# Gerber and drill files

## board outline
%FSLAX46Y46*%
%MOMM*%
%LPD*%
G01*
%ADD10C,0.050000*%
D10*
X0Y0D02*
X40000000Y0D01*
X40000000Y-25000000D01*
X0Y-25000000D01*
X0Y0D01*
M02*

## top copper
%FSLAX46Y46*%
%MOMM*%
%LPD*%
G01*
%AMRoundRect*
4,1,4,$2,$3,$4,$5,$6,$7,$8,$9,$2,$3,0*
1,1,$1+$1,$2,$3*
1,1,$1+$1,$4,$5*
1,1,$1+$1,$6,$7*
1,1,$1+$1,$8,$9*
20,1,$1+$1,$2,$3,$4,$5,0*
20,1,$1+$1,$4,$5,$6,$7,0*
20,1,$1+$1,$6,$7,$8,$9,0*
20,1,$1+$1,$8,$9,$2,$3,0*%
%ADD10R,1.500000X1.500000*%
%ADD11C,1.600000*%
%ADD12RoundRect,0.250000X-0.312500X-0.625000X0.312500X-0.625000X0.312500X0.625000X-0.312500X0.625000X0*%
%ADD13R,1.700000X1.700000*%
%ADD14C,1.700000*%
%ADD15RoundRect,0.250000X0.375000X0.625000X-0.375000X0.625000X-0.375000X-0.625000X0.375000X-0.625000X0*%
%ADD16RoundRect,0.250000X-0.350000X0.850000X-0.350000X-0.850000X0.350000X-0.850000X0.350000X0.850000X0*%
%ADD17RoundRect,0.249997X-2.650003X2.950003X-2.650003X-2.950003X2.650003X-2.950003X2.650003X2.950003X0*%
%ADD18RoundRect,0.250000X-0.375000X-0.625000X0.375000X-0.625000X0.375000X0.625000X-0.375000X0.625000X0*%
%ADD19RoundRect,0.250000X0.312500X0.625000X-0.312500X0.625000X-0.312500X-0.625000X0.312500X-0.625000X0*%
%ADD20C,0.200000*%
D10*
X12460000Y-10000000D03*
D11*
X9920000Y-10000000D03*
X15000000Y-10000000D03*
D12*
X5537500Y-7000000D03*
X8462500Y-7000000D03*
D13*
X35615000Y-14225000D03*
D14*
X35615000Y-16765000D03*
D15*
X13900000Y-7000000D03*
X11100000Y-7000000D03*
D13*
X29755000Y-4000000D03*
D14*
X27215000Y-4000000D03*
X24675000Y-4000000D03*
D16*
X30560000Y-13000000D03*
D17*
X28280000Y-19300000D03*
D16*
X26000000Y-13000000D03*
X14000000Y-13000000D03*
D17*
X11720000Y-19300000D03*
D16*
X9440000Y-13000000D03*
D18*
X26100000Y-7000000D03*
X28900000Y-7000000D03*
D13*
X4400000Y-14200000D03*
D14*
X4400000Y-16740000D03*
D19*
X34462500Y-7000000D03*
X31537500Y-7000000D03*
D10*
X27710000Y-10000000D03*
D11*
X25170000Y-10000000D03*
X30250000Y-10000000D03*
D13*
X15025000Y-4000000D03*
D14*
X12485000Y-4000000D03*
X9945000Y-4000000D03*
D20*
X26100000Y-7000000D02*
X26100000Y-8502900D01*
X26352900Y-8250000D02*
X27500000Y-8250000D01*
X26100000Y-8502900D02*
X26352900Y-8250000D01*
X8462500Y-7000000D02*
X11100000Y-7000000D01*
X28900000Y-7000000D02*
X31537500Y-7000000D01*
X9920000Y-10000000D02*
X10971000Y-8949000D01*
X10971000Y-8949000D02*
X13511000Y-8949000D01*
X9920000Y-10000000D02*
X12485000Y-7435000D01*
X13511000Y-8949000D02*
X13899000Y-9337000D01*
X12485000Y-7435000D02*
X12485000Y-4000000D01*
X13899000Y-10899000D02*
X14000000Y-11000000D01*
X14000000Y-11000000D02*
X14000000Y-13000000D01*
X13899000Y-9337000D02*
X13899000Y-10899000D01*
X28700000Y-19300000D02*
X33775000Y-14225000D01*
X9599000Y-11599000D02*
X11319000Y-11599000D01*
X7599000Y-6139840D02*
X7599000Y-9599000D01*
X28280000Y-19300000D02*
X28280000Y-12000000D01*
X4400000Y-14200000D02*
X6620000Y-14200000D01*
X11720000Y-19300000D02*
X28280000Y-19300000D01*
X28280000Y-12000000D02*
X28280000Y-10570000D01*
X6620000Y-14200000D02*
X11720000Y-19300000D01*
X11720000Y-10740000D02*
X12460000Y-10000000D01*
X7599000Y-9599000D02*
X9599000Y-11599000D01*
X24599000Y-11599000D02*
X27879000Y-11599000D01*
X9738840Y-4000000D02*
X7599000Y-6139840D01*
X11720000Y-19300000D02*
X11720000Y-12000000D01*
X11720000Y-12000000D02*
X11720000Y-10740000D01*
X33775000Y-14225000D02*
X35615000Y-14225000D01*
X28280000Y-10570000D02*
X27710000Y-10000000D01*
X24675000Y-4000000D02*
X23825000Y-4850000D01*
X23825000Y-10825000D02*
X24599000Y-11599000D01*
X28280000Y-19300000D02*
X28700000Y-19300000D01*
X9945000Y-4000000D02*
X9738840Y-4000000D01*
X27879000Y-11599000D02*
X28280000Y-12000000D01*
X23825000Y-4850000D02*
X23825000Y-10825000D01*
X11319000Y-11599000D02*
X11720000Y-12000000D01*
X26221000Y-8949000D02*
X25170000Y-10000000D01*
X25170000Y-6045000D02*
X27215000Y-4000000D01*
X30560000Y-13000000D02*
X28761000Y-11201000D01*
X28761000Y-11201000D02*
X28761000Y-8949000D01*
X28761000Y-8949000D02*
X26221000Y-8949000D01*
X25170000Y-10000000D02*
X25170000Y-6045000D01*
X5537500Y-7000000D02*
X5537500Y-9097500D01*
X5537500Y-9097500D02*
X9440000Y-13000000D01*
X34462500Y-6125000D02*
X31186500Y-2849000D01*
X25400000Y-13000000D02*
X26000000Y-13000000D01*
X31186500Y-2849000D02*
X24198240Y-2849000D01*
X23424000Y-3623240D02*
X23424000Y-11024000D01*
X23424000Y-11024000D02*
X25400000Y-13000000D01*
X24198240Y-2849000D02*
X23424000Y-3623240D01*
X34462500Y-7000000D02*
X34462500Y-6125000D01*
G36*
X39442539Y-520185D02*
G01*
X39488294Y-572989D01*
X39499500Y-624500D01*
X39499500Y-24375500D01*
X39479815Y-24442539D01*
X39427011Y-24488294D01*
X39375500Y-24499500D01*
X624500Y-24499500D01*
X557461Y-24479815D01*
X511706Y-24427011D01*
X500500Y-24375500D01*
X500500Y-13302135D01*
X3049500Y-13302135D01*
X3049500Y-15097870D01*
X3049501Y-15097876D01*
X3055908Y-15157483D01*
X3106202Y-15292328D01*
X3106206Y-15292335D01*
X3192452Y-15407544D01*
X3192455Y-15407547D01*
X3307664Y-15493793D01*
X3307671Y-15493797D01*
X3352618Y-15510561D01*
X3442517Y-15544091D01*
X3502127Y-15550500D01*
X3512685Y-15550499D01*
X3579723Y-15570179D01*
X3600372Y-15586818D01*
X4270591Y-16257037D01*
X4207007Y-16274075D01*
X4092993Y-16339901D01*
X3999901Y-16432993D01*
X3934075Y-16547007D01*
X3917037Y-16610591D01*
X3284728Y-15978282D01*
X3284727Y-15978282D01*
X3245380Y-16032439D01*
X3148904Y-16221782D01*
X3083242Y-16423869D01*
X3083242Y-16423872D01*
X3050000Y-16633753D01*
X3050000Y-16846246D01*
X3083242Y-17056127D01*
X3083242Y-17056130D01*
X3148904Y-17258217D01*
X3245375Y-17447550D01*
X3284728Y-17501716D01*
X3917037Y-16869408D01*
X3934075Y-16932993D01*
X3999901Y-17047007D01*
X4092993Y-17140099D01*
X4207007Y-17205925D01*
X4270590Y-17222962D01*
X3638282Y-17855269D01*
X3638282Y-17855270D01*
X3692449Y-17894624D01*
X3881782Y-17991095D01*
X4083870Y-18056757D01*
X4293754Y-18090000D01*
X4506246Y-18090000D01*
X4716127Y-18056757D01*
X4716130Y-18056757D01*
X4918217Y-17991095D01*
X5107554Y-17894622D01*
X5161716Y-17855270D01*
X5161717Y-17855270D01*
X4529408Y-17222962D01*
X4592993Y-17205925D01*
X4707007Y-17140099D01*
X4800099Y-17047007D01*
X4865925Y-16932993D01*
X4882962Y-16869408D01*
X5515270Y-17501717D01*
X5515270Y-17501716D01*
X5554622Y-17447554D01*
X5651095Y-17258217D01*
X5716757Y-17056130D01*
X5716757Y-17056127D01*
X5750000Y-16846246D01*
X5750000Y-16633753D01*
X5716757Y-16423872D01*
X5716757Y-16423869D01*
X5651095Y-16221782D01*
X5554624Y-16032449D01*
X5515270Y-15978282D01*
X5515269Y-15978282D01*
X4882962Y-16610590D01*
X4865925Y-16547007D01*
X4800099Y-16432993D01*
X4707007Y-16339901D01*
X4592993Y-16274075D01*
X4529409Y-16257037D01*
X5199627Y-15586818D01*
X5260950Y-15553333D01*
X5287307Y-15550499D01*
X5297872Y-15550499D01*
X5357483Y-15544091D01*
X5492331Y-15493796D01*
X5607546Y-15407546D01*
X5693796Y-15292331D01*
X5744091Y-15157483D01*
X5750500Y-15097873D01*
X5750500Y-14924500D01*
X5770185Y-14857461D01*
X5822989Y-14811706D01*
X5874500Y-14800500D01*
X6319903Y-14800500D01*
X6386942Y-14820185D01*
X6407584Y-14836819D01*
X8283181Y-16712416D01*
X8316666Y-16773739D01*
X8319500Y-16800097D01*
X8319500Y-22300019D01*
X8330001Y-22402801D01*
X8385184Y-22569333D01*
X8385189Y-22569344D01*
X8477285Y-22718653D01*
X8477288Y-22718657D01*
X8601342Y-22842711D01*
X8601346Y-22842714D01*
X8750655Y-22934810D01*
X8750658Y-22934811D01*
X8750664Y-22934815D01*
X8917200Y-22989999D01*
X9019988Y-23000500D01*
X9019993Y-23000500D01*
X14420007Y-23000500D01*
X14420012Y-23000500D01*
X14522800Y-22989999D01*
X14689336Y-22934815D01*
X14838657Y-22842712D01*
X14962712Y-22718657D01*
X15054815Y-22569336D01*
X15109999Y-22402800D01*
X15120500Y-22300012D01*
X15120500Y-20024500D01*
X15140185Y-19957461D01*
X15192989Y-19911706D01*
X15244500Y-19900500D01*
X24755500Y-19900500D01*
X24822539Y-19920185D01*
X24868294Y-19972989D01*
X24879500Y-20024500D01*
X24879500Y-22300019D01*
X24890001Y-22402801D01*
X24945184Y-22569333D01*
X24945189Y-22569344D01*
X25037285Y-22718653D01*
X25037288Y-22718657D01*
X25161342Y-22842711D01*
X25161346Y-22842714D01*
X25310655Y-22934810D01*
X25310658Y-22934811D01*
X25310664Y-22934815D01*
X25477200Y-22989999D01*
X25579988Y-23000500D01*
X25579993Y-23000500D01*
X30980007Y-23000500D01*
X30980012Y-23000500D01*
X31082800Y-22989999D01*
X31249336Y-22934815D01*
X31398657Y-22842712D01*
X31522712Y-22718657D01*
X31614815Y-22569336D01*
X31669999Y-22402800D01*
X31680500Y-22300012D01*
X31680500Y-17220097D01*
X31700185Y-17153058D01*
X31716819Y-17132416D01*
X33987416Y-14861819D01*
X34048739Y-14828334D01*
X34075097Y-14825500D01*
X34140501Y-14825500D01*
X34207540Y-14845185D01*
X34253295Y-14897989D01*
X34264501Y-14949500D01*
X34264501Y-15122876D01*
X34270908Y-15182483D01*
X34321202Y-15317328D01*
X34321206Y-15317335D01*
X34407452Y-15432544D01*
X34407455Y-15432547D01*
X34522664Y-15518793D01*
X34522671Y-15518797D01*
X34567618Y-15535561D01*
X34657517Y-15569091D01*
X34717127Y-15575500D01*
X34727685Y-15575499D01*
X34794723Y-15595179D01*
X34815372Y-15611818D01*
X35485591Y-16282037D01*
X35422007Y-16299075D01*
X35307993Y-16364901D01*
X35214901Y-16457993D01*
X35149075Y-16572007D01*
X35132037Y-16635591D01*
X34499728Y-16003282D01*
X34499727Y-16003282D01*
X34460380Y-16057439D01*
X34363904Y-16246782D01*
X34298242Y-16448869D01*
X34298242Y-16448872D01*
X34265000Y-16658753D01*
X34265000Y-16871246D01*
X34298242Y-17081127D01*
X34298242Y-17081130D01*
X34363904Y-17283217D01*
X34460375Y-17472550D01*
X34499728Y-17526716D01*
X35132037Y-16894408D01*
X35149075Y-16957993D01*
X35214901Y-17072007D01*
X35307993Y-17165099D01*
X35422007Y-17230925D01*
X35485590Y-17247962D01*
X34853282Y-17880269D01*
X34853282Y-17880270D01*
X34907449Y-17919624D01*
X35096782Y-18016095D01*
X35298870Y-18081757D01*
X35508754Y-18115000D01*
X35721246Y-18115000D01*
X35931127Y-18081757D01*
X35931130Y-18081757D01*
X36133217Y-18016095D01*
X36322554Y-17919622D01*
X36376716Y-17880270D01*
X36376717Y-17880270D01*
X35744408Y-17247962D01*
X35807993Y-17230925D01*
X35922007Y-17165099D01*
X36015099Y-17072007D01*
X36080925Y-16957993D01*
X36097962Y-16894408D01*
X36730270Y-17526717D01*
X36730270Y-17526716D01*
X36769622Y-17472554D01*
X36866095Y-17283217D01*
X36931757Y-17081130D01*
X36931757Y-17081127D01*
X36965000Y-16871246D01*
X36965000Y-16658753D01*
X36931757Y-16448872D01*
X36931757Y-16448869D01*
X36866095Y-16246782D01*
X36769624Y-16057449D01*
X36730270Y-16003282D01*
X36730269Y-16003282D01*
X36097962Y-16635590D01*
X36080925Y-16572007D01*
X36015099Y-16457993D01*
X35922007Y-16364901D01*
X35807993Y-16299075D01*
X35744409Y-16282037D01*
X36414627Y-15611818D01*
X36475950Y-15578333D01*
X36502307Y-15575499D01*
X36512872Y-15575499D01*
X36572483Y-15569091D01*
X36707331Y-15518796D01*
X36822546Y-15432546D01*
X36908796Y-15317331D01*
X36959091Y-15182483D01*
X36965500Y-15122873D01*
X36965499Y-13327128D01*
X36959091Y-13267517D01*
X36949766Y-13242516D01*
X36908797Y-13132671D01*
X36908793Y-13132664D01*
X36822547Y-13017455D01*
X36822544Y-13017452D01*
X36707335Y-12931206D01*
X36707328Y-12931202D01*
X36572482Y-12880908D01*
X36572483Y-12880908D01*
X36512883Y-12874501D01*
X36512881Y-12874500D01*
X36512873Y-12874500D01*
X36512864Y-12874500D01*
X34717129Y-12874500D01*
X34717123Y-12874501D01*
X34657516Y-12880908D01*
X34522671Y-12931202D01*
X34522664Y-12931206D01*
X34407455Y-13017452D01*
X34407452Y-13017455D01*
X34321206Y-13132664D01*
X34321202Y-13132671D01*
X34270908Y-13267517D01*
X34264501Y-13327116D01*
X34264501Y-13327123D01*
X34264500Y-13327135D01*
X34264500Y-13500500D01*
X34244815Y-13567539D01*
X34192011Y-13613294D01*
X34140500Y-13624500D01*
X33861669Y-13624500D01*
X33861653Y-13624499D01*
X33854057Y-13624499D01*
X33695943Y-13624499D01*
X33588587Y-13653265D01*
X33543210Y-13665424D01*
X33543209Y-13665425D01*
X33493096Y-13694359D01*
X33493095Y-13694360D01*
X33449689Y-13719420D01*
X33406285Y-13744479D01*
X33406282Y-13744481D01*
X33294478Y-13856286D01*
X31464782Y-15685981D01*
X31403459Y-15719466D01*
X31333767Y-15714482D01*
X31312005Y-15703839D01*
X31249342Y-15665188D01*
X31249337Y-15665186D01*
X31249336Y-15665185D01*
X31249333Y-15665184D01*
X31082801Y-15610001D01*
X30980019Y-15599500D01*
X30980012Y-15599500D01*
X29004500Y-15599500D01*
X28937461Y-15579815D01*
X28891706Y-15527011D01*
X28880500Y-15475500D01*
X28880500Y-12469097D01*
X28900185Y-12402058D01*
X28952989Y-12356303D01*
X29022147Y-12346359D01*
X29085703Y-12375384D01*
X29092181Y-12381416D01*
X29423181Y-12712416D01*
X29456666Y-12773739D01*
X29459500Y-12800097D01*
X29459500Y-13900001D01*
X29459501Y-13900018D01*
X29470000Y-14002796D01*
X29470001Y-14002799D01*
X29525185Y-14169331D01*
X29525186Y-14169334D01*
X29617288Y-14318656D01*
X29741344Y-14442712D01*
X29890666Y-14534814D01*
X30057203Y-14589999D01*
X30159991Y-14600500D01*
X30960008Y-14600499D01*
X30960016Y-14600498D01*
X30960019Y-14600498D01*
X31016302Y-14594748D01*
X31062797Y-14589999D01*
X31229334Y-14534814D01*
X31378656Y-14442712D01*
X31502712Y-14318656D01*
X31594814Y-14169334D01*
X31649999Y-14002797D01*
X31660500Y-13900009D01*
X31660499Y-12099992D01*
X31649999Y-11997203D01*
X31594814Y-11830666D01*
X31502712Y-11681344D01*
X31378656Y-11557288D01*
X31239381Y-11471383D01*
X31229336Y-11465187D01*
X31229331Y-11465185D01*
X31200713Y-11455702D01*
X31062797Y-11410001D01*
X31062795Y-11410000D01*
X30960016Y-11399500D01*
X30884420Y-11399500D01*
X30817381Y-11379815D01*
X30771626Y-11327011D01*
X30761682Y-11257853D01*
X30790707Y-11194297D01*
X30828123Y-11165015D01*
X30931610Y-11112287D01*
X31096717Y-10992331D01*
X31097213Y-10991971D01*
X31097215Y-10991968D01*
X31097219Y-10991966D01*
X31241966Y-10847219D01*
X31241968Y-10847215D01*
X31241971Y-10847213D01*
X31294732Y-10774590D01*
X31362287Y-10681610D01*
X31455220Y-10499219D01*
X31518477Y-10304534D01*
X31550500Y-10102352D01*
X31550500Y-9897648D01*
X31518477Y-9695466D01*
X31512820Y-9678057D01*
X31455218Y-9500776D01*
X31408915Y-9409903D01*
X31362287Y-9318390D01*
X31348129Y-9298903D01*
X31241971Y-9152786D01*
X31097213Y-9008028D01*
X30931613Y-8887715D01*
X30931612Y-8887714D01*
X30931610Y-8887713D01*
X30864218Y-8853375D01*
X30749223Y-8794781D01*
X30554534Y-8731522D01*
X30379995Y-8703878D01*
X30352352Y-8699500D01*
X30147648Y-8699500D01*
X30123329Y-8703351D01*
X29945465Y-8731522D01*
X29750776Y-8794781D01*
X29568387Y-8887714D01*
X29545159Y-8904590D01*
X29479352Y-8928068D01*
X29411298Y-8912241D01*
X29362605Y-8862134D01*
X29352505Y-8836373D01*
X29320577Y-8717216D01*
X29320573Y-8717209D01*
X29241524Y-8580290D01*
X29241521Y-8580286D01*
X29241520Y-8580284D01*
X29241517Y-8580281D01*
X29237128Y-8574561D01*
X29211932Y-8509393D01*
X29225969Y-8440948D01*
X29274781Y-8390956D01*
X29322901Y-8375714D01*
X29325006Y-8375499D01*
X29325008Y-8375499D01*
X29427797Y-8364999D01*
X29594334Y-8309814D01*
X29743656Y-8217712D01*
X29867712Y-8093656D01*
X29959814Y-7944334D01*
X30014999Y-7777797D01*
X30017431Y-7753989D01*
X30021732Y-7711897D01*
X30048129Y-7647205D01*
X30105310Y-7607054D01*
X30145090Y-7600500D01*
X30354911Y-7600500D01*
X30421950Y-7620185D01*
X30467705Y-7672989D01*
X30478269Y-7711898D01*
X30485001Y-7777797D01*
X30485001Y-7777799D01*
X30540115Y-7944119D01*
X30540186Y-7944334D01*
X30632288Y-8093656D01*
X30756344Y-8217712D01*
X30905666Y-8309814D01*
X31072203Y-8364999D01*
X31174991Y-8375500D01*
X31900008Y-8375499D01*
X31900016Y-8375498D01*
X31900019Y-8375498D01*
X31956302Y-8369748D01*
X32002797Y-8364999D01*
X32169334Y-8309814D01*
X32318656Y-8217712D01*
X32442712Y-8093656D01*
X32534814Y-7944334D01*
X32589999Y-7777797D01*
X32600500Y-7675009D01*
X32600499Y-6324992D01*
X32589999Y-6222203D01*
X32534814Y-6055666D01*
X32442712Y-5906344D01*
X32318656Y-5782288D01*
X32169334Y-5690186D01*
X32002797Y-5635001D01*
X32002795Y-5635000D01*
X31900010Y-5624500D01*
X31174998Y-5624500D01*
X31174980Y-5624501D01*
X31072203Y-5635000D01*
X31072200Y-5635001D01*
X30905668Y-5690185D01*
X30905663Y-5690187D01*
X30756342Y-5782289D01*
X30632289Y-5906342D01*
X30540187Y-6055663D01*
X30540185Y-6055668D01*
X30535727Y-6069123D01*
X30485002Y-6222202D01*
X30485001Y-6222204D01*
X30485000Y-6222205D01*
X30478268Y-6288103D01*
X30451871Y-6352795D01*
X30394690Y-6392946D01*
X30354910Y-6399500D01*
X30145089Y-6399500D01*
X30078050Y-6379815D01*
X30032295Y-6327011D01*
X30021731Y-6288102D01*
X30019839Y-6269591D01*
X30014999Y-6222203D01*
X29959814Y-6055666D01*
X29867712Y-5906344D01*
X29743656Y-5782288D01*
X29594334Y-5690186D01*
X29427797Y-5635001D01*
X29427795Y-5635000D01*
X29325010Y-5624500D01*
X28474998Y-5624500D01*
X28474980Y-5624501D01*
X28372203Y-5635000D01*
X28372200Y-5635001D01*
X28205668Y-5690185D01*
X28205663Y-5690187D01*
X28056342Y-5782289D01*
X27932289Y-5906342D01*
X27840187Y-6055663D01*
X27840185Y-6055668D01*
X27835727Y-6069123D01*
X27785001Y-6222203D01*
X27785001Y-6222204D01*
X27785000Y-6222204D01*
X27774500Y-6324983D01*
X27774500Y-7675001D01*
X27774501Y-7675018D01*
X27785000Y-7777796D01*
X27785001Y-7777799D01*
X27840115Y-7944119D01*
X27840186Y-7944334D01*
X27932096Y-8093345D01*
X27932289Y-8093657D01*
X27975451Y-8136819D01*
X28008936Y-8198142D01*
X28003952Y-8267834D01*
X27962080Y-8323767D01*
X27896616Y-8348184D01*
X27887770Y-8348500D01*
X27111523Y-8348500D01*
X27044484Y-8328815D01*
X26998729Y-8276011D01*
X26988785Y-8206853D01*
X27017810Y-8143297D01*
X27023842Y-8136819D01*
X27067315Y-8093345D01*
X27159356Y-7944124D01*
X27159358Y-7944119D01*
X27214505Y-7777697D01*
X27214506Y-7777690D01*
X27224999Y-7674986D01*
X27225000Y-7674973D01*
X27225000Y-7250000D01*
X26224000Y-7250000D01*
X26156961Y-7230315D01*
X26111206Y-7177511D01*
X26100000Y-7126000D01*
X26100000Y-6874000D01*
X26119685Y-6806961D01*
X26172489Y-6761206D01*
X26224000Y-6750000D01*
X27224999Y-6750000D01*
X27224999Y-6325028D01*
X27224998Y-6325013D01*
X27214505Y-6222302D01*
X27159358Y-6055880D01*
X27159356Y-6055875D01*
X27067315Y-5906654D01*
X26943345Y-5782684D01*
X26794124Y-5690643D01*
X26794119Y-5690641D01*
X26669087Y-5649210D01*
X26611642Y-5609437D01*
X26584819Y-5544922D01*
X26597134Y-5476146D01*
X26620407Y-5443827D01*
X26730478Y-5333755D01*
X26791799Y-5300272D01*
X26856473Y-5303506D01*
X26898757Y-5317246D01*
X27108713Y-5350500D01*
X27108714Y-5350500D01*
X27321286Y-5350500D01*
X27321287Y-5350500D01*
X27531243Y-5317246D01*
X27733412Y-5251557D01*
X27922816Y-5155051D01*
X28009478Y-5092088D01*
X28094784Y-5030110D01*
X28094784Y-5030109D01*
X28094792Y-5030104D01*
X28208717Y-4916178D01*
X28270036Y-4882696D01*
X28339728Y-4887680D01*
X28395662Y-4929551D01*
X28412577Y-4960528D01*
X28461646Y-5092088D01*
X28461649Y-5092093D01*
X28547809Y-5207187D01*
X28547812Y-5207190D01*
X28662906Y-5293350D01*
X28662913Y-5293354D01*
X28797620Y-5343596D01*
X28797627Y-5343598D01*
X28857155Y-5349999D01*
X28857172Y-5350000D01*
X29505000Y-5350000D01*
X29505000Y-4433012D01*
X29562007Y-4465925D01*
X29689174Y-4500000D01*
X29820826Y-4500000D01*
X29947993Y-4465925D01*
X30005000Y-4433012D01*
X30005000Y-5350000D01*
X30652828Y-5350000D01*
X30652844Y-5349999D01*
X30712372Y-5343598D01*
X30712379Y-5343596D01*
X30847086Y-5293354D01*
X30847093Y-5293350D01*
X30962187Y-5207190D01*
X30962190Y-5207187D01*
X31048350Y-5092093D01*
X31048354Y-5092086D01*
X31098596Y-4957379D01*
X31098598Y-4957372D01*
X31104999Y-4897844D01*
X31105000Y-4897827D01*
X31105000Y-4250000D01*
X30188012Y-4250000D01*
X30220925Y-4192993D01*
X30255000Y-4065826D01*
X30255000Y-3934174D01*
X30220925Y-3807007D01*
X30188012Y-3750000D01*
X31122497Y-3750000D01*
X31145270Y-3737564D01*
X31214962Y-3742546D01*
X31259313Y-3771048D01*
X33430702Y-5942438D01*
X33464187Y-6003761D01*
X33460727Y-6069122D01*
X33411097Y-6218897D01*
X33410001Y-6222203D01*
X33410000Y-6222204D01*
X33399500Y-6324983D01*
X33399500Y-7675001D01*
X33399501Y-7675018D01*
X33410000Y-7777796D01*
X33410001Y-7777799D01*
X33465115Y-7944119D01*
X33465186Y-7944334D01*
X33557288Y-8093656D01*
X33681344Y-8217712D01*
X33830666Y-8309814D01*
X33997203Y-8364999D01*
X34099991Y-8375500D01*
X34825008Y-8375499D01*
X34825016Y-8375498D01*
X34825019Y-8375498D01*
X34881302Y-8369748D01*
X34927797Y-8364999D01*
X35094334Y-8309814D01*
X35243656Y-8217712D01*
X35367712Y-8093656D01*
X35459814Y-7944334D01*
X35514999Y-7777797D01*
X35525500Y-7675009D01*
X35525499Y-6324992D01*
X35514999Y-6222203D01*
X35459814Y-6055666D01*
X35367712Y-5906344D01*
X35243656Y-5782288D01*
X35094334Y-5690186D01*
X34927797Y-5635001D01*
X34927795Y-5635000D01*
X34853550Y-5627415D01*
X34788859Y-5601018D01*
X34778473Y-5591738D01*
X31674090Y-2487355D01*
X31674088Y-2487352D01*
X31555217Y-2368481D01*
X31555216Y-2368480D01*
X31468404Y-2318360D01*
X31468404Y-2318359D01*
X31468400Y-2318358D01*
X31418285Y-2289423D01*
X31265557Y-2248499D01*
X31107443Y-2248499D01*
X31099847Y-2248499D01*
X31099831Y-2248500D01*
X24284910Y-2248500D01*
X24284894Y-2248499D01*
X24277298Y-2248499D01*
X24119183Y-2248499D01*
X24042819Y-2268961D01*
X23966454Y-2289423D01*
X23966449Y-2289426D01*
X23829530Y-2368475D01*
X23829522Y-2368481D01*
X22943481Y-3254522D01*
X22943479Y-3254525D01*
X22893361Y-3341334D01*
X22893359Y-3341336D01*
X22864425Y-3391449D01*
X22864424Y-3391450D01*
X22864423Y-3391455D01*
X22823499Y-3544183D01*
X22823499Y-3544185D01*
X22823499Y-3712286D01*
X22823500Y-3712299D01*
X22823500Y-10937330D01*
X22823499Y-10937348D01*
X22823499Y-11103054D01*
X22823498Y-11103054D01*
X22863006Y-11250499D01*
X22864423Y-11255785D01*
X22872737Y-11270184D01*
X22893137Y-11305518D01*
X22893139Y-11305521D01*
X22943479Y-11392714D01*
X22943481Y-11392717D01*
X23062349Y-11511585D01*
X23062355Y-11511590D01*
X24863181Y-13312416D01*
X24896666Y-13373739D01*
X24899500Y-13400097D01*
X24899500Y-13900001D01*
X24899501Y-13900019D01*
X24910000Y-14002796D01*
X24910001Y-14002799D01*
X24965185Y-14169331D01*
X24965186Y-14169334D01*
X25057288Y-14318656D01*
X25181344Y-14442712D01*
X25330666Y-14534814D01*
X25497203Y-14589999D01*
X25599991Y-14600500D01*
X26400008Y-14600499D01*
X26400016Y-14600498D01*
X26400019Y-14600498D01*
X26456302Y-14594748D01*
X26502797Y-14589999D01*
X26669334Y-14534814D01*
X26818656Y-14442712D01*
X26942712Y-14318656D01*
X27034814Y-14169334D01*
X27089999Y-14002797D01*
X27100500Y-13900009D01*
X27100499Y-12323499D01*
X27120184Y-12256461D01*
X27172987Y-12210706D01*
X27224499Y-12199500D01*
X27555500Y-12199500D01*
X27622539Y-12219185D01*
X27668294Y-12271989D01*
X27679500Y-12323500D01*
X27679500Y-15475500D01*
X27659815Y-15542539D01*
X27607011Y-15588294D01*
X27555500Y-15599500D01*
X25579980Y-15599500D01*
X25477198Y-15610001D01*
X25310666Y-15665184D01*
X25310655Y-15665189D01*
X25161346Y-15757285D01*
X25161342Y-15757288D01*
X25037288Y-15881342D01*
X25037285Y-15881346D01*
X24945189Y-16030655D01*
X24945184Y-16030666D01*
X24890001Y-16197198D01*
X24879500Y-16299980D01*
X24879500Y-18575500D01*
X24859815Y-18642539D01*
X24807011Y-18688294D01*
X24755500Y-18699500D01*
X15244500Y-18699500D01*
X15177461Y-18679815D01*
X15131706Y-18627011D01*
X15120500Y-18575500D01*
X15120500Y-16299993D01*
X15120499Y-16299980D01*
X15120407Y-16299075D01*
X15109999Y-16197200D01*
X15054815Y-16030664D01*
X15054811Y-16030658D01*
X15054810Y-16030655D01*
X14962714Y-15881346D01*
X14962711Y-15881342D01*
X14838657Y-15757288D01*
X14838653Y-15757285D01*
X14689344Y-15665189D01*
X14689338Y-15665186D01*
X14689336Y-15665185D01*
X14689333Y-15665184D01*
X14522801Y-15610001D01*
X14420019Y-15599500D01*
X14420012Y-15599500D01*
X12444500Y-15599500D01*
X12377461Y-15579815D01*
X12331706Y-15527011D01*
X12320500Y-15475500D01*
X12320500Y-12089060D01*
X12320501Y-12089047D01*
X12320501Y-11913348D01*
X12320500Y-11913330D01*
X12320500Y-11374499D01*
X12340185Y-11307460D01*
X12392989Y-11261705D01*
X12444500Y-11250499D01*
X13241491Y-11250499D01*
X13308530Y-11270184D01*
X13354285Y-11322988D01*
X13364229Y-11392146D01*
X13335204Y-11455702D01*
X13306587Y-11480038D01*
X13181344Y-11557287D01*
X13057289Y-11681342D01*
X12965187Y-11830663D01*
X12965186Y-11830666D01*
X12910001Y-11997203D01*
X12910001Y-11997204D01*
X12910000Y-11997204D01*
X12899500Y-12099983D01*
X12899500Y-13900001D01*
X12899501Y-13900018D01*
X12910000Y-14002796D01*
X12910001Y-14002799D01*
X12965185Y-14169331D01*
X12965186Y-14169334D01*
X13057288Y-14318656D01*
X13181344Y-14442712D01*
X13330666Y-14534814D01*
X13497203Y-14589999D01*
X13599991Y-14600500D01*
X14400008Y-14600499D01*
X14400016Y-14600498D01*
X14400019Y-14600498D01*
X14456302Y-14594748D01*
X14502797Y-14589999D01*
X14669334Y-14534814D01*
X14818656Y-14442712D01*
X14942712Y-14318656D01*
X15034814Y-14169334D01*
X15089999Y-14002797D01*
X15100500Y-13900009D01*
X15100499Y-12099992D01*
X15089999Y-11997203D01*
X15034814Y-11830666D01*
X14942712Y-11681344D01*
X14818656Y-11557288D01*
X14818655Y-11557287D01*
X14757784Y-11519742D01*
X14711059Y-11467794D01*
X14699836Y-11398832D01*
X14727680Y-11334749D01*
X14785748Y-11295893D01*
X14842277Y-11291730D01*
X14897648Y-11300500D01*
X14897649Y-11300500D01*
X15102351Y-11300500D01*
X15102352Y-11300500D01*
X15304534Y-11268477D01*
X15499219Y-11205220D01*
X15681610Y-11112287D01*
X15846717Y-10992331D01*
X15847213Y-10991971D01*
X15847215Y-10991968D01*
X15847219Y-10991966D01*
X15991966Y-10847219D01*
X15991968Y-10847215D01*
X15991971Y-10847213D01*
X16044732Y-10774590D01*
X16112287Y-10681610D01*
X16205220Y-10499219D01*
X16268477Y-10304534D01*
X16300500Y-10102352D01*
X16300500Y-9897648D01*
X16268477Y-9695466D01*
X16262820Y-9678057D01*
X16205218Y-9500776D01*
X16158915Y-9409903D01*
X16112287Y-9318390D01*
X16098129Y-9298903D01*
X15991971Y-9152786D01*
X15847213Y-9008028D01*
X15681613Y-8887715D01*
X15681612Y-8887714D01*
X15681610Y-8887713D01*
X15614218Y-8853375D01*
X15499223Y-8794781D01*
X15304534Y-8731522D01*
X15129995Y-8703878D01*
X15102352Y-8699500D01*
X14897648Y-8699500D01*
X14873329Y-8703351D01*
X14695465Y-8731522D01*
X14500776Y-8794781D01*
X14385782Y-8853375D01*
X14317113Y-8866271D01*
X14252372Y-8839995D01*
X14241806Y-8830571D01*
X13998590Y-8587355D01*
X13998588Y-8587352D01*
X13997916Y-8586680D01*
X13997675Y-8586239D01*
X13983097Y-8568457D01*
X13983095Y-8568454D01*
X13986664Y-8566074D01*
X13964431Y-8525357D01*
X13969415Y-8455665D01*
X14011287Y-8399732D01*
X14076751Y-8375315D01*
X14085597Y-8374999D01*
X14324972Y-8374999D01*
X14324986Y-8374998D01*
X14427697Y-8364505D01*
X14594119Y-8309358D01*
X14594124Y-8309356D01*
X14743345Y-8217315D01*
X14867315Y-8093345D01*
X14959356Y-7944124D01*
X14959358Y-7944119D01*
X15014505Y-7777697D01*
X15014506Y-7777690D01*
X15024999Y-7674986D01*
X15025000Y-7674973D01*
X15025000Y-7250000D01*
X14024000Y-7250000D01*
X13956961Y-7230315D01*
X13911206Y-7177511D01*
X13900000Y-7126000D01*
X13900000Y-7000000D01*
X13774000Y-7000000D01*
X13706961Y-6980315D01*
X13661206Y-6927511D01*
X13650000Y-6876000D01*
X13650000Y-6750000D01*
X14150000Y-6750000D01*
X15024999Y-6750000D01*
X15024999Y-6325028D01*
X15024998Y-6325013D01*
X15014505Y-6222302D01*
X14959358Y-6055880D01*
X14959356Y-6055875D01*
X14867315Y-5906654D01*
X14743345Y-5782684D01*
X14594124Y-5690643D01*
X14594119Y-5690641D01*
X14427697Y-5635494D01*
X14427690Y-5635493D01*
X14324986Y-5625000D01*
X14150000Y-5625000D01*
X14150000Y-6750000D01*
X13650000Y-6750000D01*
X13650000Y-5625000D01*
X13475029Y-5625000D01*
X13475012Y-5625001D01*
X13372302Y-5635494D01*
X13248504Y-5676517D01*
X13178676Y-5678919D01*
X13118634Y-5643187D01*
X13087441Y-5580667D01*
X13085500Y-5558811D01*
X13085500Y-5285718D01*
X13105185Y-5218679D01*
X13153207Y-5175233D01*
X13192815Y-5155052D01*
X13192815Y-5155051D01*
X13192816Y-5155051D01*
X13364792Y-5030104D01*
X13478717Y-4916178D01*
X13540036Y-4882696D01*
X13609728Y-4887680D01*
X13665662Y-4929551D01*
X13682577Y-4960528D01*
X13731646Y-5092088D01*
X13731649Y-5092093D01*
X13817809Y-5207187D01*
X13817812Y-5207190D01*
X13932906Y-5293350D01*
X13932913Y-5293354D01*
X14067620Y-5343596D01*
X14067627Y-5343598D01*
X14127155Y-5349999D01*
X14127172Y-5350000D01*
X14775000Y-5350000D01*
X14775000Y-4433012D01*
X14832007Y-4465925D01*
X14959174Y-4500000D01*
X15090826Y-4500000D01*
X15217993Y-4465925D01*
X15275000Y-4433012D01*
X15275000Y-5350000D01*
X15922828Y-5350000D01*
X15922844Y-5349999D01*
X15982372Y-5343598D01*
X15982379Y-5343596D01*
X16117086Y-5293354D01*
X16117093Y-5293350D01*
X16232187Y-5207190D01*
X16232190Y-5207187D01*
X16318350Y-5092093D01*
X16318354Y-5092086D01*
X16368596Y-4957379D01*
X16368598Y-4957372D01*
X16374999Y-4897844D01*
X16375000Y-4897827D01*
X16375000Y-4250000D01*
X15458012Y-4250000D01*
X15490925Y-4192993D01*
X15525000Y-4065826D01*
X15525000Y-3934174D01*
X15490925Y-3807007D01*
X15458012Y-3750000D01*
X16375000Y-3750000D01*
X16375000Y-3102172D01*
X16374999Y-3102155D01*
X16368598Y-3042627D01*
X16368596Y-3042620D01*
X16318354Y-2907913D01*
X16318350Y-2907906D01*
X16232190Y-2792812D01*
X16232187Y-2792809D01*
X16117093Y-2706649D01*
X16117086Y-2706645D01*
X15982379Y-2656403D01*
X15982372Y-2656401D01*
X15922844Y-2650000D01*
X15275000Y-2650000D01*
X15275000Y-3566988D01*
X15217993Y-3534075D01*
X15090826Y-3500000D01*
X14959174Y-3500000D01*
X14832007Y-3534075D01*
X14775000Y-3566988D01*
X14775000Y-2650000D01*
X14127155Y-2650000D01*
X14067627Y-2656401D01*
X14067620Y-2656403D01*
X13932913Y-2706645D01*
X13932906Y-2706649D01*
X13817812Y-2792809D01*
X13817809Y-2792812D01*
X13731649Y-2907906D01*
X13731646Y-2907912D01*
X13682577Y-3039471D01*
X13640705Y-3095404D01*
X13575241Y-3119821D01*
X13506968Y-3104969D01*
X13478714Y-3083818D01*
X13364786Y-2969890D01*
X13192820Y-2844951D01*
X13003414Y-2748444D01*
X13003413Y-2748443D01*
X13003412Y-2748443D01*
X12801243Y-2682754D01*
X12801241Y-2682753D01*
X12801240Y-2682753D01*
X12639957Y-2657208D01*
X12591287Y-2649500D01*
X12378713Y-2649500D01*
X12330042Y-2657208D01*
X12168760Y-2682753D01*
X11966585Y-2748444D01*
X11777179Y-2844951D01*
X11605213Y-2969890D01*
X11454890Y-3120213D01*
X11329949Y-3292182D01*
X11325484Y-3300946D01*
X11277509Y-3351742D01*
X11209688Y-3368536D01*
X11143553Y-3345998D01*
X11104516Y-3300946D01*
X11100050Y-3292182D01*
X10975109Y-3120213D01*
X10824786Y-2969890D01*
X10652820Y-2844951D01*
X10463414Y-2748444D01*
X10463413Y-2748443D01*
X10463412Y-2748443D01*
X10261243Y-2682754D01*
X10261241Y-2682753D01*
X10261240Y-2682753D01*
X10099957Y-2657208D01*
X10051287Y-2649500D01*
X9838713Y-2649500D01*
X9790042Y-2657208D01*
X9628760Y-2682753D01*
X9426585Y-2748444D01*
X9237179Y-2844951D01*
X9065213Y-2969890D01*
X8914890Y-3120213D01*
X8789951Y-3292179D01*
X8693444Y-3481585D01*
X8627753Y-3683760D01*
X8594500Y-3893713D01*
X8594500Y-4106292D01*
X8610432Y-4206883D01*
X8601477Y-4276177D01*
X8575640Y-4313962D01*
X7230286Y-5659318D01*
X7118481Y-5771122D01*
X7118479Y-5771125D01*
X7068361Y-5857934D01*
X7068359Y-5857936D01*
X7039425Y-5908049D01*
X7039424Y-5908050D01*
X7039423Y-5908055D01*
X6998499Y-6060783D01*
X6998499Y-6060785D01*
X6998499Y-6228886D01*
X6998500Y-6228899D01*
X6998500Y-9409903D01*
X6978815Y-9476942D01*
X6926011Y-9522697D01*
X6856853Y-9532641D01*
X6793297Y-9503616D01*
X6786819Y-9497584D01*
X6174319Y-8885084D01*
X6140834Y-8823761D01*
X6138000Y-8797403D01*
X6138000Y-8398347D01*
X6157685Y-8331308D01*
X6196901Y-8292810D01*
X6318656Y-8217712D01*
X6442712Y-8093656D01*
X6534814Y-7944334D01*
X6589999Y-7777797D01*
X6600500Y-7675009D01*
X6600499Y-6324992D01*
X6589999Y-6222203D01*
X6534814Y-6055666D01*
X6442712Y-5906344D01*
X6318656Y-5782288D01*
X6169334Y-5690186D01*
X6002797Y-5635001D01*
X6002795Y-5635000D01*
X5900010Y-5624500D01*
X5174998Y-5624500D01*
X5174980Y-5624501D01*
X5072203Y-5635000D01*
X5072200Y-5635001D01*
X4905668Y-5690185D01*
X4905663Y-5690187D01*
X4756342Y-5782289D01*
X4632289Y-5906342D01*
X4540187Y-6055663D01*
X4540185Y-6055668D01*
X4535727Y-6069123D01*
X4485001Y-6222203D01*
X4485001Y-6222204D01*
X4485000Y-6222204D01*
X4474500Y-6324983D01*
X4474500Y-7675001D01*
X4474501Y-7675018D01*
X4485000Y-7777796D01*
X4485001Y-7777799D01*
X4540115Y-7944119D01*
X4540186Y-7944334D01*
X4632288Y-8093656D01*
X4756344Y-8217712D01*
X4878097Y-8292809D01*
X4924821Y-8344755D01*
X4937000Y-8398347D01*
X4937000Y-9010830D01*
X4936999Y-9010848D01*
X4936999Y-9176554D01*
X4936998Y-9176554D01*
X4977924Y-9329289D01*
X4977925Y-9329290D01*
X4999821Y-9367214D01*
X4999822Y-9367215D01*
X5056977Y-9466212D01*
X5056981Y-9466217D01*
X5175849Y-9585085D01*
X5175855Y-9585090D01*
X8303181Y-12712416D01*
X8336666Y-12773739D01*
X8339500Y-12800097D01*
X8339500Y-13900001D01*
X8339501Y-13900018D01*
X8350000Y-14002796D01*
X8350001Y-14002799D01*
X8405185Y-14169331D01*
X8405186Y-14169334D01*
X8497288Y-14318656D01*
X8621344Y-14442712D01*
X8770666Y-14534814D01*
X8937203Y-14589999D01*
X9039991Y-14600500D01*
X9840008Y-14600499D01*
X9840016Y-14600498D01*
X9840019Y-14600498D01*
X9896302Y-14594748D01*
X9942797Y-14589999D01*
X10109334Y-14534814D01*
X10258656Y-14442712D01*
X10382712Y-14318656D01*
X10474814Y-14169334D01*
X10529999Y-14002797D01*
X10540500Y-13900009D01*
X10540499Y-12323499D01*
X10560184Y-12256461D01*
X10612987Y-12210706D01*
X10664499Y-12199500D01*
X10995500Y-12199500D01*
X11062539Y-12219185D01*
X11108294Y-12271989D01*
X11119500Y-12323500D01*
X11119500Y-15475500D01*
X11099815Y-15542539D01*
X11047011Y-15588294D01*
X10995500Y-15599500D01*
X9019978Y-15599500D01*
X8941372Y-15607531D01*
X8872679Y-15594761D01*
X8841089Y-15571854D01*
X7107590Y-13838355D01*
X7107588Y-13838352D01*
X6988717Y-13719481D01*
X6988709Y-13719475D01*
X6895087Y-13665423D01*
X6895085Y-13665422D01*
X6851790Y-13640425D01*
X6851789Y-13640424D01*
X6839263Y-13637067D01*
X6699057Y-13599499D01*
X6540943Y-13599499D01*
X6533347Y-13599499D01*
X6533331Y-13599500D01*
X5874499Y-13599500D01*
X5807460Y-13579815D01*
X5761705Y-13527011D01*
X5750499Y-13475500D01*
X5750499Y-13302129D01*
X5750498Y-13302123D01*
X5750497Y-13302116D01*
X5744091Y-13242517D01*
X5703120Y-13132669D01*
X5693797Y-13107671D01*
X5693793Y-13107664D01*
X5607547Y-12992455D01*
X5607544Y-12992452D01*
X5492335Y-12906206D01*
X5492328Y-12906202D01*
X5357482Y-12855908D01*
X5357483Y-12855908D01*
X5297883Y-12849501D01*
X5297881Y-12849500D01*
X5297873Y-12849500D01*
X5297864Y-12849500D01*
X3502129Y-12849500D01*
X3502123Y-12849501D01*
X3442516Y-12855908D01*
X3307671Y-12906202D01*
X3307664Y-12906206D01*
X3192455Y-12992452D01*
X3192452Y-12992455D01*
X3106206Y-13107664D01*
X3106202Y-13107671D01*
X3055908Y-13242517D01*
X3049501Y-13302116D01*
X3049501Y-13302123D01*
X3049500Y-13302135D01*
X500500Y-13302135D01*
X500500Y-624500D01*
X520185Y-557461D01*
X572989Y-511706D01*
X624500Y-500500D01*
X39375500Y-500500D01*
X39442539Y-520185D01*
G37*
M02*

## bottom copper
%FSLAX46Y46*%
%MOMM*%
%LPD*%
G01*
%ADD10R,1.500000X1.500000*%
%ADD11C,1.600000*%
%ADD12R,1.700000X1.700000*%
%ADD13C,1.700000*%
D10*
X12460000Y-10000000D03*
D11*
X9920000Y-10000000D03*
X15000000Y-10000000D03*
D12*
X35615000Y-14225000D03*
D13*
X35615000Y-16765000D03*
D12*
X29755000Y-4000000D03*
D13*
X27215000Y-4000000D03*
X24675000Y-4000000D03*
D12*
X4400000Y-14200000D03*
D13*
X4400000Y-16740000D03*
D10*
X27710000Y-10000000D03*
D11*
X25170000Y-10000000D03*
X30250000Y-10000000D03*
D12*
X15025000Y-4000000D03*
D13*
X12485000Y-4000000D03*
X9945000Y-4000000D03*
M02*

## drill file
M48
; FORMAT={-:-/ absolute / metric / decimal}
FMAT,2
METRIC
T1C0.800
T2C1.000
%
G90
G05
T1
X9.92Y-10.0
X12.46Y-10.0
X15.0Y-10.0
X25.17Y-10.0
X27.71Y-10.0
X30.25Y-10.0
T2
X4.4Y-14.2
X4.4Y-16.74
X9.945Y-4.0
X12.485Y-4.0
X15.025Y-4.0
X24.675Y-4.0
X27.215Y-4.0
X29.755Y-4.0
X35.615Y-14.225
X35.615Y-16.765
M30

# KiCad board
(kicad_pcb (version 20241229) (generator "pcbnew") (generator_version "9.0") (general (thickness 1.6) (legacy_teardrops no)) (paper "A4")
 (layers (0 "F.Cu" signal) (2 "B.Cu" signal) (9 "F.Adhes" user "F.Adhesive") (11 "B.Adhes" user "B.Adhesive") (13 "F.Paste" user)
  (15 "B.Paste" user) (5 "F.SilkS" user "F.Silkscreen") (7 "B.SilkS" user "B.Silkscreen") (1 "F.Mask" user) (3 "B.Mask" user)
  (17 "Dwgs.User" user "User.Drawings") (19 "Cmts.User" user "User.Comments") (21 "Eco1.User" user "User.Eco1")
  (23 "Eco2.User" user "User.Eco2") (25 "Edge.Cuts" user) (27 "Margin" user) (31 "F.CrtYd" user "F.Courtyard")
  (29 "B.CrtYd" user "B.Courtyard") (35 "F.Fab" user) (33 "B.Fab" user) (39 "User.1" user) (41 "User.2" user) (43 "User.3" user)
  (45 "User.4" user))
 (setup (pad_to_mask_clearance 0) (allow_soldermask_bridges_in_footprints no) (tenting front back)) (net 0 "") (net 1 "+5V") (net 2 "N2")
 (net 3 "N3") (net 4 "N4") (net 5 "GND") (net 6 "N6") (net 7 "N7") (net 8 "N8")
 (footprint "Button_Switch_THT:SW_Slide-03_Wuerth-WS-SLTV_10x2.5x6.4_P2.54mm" (layer "F.Cu") (at 12.46 10)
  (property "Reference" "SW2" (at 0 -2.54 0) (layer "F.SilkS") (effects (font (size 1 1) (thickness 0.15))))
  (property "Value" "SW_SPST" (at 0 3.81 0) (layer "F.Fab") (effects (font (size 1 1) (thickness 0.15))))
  (pad "1" thru_hole rect (at 0 0) (size 1.5 1.5) (drill 0.8) (layers "*.Cu" "*.Mask") (remove_unused_layers no) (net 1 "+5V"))
  (pad "2" thru_hole circle (at -2.54 0) (size 1.6 1.6) (drill 0.8) (layers "*.Cu" "*.Mask") (remove_unused_layers no) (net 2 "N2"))
  (pad "3" thru_hole circle (at 2.54 0) (size 1.6 1.6) (drill 0.8) (layers "*.Cu" "*.Mask") (remove_unused_layers no)))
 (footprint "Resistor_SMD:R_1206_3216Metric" (layer "F.Cu") (at 7 7)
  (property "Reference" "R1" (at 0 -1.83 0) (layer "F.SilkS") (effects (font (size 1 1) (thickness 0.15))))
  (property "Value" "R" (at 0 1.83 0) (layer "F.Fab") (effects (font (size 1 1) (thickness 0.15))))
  (pad "1" smd roundrect (at -1.4625 0) (size 1.125 1.75) (layers "F.Cu" "F.Mask" "F.Paste") (roundrect_rratio 0.222222) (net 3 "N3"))
  (pad "2" smd roundrect (at 1.4625 0) (size 1.125 1.75) (layers "F.Cu" "F.Mask" "F.Paste") (roundrect_rratio 0.222222) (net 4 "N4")))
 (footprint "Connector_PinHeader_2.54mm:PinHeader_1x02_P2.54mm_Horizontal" (layer "F.Cu") (at 35.615 14.225)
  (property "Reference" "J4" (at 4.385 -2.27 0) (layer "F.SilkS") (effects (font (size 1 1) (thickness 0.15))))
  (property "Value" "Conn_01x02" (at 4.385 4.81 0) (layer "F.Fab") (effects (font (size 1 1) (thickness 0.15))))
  (pad "1" thru_hole rect (at 0 0) (size 1.7 1.7) (drill 1) (layers "*.Cu" "*.Mask") (remove_unused_layers no) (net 1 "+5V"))
  (pad "2" thru_hole circle (at 0 2.54) (size 1.7 1.7) (drill 1) (layers "*.Cu" "*.Mask") (remove_unused_layers no) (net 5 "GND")))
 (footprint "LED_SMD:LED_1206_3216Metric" (layer "F.Cu") (at 12.5 7 180)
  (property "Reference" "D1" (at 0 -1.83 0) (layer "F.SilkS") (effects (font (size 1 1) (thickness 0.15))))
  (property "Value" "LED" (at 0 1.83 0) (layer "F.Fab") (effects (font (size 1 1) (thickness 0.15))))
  (pad "1" smd roundrect (at -1.4 0 180) (size 1.25 1.75) (layers "F.Cu" "F.Mask" "F.Paste") (roundrect_rratio 0.2) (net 5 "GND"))
  (pad "2" smd roundrect (at 1.4 0 180) (size 1.25 1.75) (layers "F.Cu" "F.Mask" "F.Paste") (roundrect_rratio 0.2) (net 4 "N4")))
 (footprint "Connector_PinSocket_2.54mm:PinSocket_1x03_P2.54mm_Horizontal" (layer "F.Cu") (at 29.755 4 -90)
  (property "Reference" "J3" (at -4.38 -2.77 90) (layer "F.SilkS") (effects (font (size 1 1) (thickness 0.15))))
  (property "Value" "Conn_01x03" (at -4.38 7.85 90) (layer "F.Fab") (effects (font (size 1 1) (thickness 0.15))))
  (pad "1" thru_hole rect (at 0 0 270) (size 1.7 1.7) (drill 1) (layers "*.Cu" "*.Mask") (remove_unused_layers no) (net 5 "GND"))
  (pad "2" thru_hole circle (at 0 2.54 270) (size 1.7 1.7) (drill 1) (layers "*.Cu" "*.Mask") (remove_unused_layers no) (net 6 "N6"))
  (pad "3" thru_hole circle (at 0 5.08 270) (size 1.7 1.7) (drill 1) (layers "*.Cu" "*.Mask") (remove_unused_layers no) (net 1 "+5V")))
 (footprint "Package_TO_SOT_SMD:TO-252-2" (layer "F.Cu") (at 28.28 18.04 -90)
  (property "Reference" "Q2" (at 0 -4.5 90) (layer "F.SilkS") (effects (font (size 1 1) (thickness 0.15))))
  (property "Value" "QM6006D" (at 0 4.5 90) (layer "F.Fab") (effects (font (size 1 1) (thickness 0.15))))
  (pad "" smd roundrect (at -0.415 -1.525 270) (size 3.05 2.75) (layers "F.Paste") (roundrect_rratio 0.090909))
  (pad "" smd roundrect (at -0.415 1.525 270) (size 3.05 2.75) (layers "F.Paste") (roundrect_rratio 0.090909))
  (pad "" smd roundrect (at 2.935 -1.525 270) (size 3.05 2.75) (layers "F.Paste") (roundrect_rratio 0.090909))
  (pad "" smd roundrect (at 2.935 1.525 270) (size 3.05 2.75) (layers "F.Paste") (roundrect_rratio 0.090909))
  (pad "1" smd roundrect (at -5.04 -2.28 270) (size 2.2 1.2) (layers "F.Cu" "F.Mask" "F.Paste") (roundrect_rratio 0.208333) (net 6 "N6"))
  (pad "2" smd roundrect (at 1.26 0 270) (size 6.4 5.8) (layers "F.Cu" "F.Mask") (roundrect_rratio 0.043103) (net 1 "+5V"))
  (pad "3" smd roundrect (at -5.04 2.28 270) (size 2.2 1.2) (layers "F.Cu" "F.Mask" "F.Paste") (roundrect_rratio 0.208333) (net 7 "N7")))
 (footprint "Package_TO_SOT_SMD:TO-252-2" (layer "F.Cu") (at 11.72 18.04 -90)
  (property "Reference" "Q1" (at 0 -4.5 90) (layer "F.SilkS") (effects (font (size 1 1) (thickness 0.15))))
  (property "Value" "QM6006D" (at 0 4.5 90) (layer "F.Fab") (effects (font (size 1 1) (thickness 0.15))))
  (pad "" smd roundrect (at -0.415 -1.525 270) (size 3.05 2.75) (layers "F.Paste") (roundrect_rratio 0.090909))
  (pad "" smd roundrect (at -0.415 1.525 270) (size 3.05 2.75) (layers "F.Paste") (roundrect_rratio 0.090909))
  (pad "" smd roundrect (at 2.935 -1.525 270) (size 3.05 2.75) (layers "F.Paste") (roundrect_rratio 0.090909))
  (pad "" smd roundrect (at 2.935 1.525 270) (size 3.05 2.75) (layers "F.Paste") (roundrect_rratio 0.090909))
  (pad "1" smd roundrect (at -5.04 -2.28 270) (size 2.2 1.2) (layers "F.Cu" "F.Mask" "F.Paste") (roundrect_rratio 0.208333) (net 2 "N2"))
  (pad "2" smd roundrect (at 1.26 0 270) (size 6.4 5.8) (layers "F.Cu" "F.Mask") (roundrect_rratio 0.043103) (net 1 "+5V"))
  (pad "3" smd roundrect (at -5.04 2.28 270) (size 2.2 1.2) (layers "F.Cu" "F.Mask" "F.Paste") (roundrect_rratio 0.208333) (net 3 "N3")))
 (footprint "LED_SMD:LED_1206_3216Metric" (layer "F.Cu") (at 27.5 7)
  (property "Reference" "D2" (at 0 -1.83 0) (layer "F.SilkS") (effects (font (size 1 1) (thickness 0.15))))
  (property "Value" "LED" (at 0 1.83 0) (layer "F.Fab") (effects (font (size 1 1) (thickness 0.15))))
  (pad "1" smd roundrect (at -1.4 0) (size 1.25 1.75) (layers "F.Cu" "F.Mask" "F.Paste") (roundrect_rratio 0.2) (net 5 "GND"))
  (pad "2" smd roundrect (at 1.4 0) (size 1.25 1.75) (layers "F.Cu" "F.Mask" "F.Paste") (roundrect_rratio 0.2) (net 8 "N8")))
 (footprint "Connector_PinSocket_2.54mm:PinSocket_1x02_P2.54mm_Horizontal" (layer "F.Cu") (at 4.4 14.2)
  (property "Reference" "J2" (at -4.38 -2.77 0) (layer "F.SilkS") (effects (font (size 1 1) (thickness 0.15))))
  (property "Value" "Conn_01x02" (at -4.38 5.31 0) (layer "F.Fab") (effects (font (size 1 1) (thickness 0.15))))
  (pad "1" thru_hole rect (at 0 0) (size 1.7 1.7) (drill 1) (layers "*.Cu" "*.Mask") (remove_unused_layers no) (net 1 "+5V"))
  (pad "2" thru_hole circle (at 0 2.54) (size 1.7 1.7) (drill 1) (layers "*.Cu" "*.Mask") (remove_unused_layers no) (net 5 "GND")))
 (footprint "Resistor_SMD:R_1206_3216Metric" (layer "F.Cu") (at 33 7 180)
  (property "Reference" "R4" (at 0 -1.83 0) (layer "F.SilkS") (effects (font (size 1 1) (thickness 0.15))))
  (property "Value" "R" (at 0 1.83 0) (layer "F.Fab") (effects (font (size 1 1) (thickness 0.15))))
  (pad "1" smd roundrect (at -1.4625 0 180) (size 1.125 1.75) (layers "F.Cu" "F.Mask" "F.Paste") (roundrect_rratio 0.222222) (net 7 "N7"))
  (pad "2" smd roundrect (at 1.4625 0 180) (size 1.125 1.75) (layers "F.Cu" "F.Mask" "F.Paste") (roundrect_rratio 0.222222) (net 8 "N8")))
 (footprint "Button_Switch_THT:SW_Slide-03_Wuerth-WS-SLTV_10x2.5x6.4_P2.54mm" (layer "F.Cu") (at 27.71 10)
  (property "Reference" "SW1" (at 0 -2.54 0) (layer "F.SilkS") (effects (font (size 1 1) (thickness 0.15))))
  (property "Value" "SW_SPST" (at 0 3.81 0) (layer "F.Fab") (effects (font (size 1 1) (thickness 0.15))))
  (pad "1" thru_hole rect (at 0 0) (size 1.5 1.5) (drill 0.8) (layers "*.Cu" "*.Mask") (remove_unused_layers no) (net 1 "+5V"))
  (pad "2" thru_hole circle (at -2.54 0) (size 1.6 1.6) (drill 0.8) (layers "*.Cu" "*.Mask") (remove_unused_layers no) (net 6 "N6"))
  (pad "3" thru_hole circle (at 2.54 0) (size 1.6 1.6) (drill 0.8) (layers "*.Cu" "*.Mask") (remove_unused_layers no)))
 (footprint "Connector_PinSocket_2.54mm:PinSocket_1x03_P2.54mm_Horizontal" (layer "F.Cu") (at 15.025 4 -90)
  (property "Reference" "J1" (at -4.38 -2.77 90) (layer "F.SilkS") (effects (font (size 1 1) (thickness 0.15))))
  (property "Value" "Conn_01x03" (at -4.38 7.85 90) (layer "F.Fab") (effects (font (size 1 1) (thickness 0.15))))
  (pad "1" thru_hole rect (at 0 0 270) (size 1.7 1.7) (drill 1) (layers "*.Cu" "*.Mask") (remove_unused_layers no) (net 5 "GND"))
  (pad "2" thru_hole circle (at 0 2.54 270) (size 1.7 1.7) (drill 1) (layers "*.Cu" "*.Mask") (remove_unused_layers no) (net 2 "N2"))
  (pad "3" thru_hole circle (at 0 5.08 270) (size 1.7 1.7) (drill 1) (layers "*.Cu" "*.Mask") (remove_unused_layers no) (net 1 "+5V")))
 (gr_rect (start 0 0) (end 40 25) (stroke (width 0.05) (type solid)) (fill no) (layer "Edge.Cuts"))
 (segment (start 26.1 7) (end 26.1 8.5029) (width 0.2) (layer "F.Cu") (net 5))
 (segment (start 26.3529 8.25) (end 27.5 8.25) (width 0.2) (layer "F.Cu") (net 5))
 (segment (start 26.1 8.5029) (end 26.3529 8.25) (width 0.2) (layer "F.Cu") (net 5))
 (segment (start 8.4625 7) (end 11.1 7) (width 0.2) (layer "F.Cu") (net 4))
 (segment (start 28.9 7) (end 31.5375 7) (width 0.2) (layer "F.Cu") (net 8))
 (segment (start 9.92 10) (end 10.971 8.949) (width 0.2) (layer "F.Cu") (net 2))
 (segment (start 10.971 8.949) (end 13.511 8.949) (width 0.2) (layer "F.Cu") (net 2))
 (segment (start 9.92 10) (end 12.485 7.435) (width 0.2) (layer "F.Cu") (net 2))
 (segment (start 13.511 8.949) (end 13.899 9.337) (width 0.2) (layer "F.Cu") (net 2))
 (segment (start 12.485 7.435) (end 12.485 4) (width 0.2) (layer "F.Cu") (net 2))
 (segment (start 13.899 10.899) (end 14 11) (width 0.2) (layer "F.Cu") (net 2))
 (segment (start 14 11) (end 14 13) (width 0.2) (layer "F.Cu") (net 2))
 (segment (start 13.899 9.337) (end 13.899 10.899) (width 0.2) (layer "F.Cu") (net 2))
 (segment (start 28.7 19.3) (end 33.775 14.225) (width 0.2) (layer "F.Cu") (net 1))
 (segment (start 9.599 11.599) (end 11.319 11.599) (width 0.2) (layer "F.Cu") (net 1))
 (segment (start 7.599 6.13984) (end 7.599 9.599) (width 0.2) (layer "F.Cu") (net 1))
 (segment (start 28.28 19.3) (end 28.28 12) (width 0.2) (layer "F.Cu") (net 1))
 (segment (start 4.4 14.2) (end 6.62 14.2) (width 0.2) (layer "F.Cu") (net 1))
 (segment (start 11.72 19.3) (end 28.28 19.3) (width 0.2) (layer "F.Cu") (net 1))
 (segment (start 28.28 12) (end 28.28 10.57) (width 0.2) (layer "F.Cu") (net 1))
 (segment (start 6.62 14.2) (end 11.72 19.3) (width 0.2) (layer "F.Cu") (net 1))
 (segment (start 11.72 10.74) (end 12.46 10) (width 0.2) (layer "F.Cu") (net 1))
 (segment (start 7.599 9.599) (end 9.599 11.599) (width 0.2) (layer "F.Cu") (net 1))
 (segment (start 24.599 11.599) (end 27.879 11.599) (width 0.2) (layer "F.Cu") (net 1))
 (segment (start 9.73884 4) (end 7.599 6.13984) (width 0.2) (layer "F.Cu") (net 1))
 (segment (start 11.72 19.3) (end 11.72 12) (width 0.2) (layer "F.Cu") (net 1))
 (segment (start 11.72 12) (end 11.72 10.74) (width 0.2) (layer "F.Cu") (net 1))
 (segment (start 33.775 14.225) (end 35.615 14.225) (width 0.2) (layer "F.Cu") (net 1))
 (segment (start 28.28 10.57) (end 27.71 10) (width 0.2) (layer "F.Cu") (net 1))
 (segment (start 24.675 4) (end 23.825 4.85) (width 0.2) (layer "F.Cu") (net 1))
 (segment (start 23.825 10.825) (end 24.599 11.599) (width 0.2) (layer "F.Cu") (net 1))
 (segment (start 28.28 19.3) (end 28.7 19.3) (width 0.2) (layer "F.Cu") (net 1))
 (segment (start 9.945 4) (end 9.73884 4) (width 0.2) (layer "F.Cu") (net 1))
 (segment (start 27.879 11.599) (end 28.28 12) (width 0.2) (layer "F.Cu") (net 1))
 (segment (start 23.825 4.85) (end 23.825 10.825) (width 0.2) (layer "F.Cu") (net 1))
 (segment (start 11.319 11.599) (end 11.72 12) (width 0.2) (layer "F.Cu") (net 1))
 (segment (start 26.221 8.949) (end 25.17 10) (width 0.2) (layer "F.Cu") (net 6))
 (segment (start 25.17 6.045) (end 27.215 4) (width 0.2) (layer "F.Cu") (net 6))
 (segment (start 30.56 13) (end 28.761 11.201) (width 0.2) (layer "F.Cu") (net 6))
 (segment (start 28.761 11.201) (end 28.761 8.949) (width 0.2) (layer "F.Cu") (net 6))
 (segment (start 28.761 8.949) (end 26.221 8.949) (width 0.2) (layer "F.Cu") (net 6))
 (segment (start 25.17 10) (end 25.17 6.045) (width 0.2) (layer "F.Cu") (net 6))
 (segment (start 5.5375 7) (end 5.5375 9.0975) (width 0.2) (layer "F.Cu") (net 3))
 (segment (start 5.5375 9.0975) (end 9.44 13) (width 0.2) (layer "F.Cu") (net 3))
 (segment (start 34.4625 6.125) (end 31.1865 2.849) (width 0.2) (layer "F.Cu") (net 7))
 (segment (start 25.4 13) (end 26 13) (width 0.2) (layer "F.Cu") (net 7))
 (segment (start 31.1865 2.849) (end 24.19824 2.849) (width 0.2) (layer "F.Cu") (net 7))
 (segment (start 23.424 3.62324) (end 23.424 11.024) (width 0.2) (layer "F.Cu") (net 7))
 (segment (start 23.424 11.024) (end 25.4 13) (width 0.2) (layer "F.Cu") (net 7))
 (segment (start 24.19824 2.849) (end 23.424 3.62324) (width 0.2) (layer "F.Cu") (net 7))
 (segment (start 34.4625 7) (end 34.4625 6.125) (width 0.2) (layer "F.Cu") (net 7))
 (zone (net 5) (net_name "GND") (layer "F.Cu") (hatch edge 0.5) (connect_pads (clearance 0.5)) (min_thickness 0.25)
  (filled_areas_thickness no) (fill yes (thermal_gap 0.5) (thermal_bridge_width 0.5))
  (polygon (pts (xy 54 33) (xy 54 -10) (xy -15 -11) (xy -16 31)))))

